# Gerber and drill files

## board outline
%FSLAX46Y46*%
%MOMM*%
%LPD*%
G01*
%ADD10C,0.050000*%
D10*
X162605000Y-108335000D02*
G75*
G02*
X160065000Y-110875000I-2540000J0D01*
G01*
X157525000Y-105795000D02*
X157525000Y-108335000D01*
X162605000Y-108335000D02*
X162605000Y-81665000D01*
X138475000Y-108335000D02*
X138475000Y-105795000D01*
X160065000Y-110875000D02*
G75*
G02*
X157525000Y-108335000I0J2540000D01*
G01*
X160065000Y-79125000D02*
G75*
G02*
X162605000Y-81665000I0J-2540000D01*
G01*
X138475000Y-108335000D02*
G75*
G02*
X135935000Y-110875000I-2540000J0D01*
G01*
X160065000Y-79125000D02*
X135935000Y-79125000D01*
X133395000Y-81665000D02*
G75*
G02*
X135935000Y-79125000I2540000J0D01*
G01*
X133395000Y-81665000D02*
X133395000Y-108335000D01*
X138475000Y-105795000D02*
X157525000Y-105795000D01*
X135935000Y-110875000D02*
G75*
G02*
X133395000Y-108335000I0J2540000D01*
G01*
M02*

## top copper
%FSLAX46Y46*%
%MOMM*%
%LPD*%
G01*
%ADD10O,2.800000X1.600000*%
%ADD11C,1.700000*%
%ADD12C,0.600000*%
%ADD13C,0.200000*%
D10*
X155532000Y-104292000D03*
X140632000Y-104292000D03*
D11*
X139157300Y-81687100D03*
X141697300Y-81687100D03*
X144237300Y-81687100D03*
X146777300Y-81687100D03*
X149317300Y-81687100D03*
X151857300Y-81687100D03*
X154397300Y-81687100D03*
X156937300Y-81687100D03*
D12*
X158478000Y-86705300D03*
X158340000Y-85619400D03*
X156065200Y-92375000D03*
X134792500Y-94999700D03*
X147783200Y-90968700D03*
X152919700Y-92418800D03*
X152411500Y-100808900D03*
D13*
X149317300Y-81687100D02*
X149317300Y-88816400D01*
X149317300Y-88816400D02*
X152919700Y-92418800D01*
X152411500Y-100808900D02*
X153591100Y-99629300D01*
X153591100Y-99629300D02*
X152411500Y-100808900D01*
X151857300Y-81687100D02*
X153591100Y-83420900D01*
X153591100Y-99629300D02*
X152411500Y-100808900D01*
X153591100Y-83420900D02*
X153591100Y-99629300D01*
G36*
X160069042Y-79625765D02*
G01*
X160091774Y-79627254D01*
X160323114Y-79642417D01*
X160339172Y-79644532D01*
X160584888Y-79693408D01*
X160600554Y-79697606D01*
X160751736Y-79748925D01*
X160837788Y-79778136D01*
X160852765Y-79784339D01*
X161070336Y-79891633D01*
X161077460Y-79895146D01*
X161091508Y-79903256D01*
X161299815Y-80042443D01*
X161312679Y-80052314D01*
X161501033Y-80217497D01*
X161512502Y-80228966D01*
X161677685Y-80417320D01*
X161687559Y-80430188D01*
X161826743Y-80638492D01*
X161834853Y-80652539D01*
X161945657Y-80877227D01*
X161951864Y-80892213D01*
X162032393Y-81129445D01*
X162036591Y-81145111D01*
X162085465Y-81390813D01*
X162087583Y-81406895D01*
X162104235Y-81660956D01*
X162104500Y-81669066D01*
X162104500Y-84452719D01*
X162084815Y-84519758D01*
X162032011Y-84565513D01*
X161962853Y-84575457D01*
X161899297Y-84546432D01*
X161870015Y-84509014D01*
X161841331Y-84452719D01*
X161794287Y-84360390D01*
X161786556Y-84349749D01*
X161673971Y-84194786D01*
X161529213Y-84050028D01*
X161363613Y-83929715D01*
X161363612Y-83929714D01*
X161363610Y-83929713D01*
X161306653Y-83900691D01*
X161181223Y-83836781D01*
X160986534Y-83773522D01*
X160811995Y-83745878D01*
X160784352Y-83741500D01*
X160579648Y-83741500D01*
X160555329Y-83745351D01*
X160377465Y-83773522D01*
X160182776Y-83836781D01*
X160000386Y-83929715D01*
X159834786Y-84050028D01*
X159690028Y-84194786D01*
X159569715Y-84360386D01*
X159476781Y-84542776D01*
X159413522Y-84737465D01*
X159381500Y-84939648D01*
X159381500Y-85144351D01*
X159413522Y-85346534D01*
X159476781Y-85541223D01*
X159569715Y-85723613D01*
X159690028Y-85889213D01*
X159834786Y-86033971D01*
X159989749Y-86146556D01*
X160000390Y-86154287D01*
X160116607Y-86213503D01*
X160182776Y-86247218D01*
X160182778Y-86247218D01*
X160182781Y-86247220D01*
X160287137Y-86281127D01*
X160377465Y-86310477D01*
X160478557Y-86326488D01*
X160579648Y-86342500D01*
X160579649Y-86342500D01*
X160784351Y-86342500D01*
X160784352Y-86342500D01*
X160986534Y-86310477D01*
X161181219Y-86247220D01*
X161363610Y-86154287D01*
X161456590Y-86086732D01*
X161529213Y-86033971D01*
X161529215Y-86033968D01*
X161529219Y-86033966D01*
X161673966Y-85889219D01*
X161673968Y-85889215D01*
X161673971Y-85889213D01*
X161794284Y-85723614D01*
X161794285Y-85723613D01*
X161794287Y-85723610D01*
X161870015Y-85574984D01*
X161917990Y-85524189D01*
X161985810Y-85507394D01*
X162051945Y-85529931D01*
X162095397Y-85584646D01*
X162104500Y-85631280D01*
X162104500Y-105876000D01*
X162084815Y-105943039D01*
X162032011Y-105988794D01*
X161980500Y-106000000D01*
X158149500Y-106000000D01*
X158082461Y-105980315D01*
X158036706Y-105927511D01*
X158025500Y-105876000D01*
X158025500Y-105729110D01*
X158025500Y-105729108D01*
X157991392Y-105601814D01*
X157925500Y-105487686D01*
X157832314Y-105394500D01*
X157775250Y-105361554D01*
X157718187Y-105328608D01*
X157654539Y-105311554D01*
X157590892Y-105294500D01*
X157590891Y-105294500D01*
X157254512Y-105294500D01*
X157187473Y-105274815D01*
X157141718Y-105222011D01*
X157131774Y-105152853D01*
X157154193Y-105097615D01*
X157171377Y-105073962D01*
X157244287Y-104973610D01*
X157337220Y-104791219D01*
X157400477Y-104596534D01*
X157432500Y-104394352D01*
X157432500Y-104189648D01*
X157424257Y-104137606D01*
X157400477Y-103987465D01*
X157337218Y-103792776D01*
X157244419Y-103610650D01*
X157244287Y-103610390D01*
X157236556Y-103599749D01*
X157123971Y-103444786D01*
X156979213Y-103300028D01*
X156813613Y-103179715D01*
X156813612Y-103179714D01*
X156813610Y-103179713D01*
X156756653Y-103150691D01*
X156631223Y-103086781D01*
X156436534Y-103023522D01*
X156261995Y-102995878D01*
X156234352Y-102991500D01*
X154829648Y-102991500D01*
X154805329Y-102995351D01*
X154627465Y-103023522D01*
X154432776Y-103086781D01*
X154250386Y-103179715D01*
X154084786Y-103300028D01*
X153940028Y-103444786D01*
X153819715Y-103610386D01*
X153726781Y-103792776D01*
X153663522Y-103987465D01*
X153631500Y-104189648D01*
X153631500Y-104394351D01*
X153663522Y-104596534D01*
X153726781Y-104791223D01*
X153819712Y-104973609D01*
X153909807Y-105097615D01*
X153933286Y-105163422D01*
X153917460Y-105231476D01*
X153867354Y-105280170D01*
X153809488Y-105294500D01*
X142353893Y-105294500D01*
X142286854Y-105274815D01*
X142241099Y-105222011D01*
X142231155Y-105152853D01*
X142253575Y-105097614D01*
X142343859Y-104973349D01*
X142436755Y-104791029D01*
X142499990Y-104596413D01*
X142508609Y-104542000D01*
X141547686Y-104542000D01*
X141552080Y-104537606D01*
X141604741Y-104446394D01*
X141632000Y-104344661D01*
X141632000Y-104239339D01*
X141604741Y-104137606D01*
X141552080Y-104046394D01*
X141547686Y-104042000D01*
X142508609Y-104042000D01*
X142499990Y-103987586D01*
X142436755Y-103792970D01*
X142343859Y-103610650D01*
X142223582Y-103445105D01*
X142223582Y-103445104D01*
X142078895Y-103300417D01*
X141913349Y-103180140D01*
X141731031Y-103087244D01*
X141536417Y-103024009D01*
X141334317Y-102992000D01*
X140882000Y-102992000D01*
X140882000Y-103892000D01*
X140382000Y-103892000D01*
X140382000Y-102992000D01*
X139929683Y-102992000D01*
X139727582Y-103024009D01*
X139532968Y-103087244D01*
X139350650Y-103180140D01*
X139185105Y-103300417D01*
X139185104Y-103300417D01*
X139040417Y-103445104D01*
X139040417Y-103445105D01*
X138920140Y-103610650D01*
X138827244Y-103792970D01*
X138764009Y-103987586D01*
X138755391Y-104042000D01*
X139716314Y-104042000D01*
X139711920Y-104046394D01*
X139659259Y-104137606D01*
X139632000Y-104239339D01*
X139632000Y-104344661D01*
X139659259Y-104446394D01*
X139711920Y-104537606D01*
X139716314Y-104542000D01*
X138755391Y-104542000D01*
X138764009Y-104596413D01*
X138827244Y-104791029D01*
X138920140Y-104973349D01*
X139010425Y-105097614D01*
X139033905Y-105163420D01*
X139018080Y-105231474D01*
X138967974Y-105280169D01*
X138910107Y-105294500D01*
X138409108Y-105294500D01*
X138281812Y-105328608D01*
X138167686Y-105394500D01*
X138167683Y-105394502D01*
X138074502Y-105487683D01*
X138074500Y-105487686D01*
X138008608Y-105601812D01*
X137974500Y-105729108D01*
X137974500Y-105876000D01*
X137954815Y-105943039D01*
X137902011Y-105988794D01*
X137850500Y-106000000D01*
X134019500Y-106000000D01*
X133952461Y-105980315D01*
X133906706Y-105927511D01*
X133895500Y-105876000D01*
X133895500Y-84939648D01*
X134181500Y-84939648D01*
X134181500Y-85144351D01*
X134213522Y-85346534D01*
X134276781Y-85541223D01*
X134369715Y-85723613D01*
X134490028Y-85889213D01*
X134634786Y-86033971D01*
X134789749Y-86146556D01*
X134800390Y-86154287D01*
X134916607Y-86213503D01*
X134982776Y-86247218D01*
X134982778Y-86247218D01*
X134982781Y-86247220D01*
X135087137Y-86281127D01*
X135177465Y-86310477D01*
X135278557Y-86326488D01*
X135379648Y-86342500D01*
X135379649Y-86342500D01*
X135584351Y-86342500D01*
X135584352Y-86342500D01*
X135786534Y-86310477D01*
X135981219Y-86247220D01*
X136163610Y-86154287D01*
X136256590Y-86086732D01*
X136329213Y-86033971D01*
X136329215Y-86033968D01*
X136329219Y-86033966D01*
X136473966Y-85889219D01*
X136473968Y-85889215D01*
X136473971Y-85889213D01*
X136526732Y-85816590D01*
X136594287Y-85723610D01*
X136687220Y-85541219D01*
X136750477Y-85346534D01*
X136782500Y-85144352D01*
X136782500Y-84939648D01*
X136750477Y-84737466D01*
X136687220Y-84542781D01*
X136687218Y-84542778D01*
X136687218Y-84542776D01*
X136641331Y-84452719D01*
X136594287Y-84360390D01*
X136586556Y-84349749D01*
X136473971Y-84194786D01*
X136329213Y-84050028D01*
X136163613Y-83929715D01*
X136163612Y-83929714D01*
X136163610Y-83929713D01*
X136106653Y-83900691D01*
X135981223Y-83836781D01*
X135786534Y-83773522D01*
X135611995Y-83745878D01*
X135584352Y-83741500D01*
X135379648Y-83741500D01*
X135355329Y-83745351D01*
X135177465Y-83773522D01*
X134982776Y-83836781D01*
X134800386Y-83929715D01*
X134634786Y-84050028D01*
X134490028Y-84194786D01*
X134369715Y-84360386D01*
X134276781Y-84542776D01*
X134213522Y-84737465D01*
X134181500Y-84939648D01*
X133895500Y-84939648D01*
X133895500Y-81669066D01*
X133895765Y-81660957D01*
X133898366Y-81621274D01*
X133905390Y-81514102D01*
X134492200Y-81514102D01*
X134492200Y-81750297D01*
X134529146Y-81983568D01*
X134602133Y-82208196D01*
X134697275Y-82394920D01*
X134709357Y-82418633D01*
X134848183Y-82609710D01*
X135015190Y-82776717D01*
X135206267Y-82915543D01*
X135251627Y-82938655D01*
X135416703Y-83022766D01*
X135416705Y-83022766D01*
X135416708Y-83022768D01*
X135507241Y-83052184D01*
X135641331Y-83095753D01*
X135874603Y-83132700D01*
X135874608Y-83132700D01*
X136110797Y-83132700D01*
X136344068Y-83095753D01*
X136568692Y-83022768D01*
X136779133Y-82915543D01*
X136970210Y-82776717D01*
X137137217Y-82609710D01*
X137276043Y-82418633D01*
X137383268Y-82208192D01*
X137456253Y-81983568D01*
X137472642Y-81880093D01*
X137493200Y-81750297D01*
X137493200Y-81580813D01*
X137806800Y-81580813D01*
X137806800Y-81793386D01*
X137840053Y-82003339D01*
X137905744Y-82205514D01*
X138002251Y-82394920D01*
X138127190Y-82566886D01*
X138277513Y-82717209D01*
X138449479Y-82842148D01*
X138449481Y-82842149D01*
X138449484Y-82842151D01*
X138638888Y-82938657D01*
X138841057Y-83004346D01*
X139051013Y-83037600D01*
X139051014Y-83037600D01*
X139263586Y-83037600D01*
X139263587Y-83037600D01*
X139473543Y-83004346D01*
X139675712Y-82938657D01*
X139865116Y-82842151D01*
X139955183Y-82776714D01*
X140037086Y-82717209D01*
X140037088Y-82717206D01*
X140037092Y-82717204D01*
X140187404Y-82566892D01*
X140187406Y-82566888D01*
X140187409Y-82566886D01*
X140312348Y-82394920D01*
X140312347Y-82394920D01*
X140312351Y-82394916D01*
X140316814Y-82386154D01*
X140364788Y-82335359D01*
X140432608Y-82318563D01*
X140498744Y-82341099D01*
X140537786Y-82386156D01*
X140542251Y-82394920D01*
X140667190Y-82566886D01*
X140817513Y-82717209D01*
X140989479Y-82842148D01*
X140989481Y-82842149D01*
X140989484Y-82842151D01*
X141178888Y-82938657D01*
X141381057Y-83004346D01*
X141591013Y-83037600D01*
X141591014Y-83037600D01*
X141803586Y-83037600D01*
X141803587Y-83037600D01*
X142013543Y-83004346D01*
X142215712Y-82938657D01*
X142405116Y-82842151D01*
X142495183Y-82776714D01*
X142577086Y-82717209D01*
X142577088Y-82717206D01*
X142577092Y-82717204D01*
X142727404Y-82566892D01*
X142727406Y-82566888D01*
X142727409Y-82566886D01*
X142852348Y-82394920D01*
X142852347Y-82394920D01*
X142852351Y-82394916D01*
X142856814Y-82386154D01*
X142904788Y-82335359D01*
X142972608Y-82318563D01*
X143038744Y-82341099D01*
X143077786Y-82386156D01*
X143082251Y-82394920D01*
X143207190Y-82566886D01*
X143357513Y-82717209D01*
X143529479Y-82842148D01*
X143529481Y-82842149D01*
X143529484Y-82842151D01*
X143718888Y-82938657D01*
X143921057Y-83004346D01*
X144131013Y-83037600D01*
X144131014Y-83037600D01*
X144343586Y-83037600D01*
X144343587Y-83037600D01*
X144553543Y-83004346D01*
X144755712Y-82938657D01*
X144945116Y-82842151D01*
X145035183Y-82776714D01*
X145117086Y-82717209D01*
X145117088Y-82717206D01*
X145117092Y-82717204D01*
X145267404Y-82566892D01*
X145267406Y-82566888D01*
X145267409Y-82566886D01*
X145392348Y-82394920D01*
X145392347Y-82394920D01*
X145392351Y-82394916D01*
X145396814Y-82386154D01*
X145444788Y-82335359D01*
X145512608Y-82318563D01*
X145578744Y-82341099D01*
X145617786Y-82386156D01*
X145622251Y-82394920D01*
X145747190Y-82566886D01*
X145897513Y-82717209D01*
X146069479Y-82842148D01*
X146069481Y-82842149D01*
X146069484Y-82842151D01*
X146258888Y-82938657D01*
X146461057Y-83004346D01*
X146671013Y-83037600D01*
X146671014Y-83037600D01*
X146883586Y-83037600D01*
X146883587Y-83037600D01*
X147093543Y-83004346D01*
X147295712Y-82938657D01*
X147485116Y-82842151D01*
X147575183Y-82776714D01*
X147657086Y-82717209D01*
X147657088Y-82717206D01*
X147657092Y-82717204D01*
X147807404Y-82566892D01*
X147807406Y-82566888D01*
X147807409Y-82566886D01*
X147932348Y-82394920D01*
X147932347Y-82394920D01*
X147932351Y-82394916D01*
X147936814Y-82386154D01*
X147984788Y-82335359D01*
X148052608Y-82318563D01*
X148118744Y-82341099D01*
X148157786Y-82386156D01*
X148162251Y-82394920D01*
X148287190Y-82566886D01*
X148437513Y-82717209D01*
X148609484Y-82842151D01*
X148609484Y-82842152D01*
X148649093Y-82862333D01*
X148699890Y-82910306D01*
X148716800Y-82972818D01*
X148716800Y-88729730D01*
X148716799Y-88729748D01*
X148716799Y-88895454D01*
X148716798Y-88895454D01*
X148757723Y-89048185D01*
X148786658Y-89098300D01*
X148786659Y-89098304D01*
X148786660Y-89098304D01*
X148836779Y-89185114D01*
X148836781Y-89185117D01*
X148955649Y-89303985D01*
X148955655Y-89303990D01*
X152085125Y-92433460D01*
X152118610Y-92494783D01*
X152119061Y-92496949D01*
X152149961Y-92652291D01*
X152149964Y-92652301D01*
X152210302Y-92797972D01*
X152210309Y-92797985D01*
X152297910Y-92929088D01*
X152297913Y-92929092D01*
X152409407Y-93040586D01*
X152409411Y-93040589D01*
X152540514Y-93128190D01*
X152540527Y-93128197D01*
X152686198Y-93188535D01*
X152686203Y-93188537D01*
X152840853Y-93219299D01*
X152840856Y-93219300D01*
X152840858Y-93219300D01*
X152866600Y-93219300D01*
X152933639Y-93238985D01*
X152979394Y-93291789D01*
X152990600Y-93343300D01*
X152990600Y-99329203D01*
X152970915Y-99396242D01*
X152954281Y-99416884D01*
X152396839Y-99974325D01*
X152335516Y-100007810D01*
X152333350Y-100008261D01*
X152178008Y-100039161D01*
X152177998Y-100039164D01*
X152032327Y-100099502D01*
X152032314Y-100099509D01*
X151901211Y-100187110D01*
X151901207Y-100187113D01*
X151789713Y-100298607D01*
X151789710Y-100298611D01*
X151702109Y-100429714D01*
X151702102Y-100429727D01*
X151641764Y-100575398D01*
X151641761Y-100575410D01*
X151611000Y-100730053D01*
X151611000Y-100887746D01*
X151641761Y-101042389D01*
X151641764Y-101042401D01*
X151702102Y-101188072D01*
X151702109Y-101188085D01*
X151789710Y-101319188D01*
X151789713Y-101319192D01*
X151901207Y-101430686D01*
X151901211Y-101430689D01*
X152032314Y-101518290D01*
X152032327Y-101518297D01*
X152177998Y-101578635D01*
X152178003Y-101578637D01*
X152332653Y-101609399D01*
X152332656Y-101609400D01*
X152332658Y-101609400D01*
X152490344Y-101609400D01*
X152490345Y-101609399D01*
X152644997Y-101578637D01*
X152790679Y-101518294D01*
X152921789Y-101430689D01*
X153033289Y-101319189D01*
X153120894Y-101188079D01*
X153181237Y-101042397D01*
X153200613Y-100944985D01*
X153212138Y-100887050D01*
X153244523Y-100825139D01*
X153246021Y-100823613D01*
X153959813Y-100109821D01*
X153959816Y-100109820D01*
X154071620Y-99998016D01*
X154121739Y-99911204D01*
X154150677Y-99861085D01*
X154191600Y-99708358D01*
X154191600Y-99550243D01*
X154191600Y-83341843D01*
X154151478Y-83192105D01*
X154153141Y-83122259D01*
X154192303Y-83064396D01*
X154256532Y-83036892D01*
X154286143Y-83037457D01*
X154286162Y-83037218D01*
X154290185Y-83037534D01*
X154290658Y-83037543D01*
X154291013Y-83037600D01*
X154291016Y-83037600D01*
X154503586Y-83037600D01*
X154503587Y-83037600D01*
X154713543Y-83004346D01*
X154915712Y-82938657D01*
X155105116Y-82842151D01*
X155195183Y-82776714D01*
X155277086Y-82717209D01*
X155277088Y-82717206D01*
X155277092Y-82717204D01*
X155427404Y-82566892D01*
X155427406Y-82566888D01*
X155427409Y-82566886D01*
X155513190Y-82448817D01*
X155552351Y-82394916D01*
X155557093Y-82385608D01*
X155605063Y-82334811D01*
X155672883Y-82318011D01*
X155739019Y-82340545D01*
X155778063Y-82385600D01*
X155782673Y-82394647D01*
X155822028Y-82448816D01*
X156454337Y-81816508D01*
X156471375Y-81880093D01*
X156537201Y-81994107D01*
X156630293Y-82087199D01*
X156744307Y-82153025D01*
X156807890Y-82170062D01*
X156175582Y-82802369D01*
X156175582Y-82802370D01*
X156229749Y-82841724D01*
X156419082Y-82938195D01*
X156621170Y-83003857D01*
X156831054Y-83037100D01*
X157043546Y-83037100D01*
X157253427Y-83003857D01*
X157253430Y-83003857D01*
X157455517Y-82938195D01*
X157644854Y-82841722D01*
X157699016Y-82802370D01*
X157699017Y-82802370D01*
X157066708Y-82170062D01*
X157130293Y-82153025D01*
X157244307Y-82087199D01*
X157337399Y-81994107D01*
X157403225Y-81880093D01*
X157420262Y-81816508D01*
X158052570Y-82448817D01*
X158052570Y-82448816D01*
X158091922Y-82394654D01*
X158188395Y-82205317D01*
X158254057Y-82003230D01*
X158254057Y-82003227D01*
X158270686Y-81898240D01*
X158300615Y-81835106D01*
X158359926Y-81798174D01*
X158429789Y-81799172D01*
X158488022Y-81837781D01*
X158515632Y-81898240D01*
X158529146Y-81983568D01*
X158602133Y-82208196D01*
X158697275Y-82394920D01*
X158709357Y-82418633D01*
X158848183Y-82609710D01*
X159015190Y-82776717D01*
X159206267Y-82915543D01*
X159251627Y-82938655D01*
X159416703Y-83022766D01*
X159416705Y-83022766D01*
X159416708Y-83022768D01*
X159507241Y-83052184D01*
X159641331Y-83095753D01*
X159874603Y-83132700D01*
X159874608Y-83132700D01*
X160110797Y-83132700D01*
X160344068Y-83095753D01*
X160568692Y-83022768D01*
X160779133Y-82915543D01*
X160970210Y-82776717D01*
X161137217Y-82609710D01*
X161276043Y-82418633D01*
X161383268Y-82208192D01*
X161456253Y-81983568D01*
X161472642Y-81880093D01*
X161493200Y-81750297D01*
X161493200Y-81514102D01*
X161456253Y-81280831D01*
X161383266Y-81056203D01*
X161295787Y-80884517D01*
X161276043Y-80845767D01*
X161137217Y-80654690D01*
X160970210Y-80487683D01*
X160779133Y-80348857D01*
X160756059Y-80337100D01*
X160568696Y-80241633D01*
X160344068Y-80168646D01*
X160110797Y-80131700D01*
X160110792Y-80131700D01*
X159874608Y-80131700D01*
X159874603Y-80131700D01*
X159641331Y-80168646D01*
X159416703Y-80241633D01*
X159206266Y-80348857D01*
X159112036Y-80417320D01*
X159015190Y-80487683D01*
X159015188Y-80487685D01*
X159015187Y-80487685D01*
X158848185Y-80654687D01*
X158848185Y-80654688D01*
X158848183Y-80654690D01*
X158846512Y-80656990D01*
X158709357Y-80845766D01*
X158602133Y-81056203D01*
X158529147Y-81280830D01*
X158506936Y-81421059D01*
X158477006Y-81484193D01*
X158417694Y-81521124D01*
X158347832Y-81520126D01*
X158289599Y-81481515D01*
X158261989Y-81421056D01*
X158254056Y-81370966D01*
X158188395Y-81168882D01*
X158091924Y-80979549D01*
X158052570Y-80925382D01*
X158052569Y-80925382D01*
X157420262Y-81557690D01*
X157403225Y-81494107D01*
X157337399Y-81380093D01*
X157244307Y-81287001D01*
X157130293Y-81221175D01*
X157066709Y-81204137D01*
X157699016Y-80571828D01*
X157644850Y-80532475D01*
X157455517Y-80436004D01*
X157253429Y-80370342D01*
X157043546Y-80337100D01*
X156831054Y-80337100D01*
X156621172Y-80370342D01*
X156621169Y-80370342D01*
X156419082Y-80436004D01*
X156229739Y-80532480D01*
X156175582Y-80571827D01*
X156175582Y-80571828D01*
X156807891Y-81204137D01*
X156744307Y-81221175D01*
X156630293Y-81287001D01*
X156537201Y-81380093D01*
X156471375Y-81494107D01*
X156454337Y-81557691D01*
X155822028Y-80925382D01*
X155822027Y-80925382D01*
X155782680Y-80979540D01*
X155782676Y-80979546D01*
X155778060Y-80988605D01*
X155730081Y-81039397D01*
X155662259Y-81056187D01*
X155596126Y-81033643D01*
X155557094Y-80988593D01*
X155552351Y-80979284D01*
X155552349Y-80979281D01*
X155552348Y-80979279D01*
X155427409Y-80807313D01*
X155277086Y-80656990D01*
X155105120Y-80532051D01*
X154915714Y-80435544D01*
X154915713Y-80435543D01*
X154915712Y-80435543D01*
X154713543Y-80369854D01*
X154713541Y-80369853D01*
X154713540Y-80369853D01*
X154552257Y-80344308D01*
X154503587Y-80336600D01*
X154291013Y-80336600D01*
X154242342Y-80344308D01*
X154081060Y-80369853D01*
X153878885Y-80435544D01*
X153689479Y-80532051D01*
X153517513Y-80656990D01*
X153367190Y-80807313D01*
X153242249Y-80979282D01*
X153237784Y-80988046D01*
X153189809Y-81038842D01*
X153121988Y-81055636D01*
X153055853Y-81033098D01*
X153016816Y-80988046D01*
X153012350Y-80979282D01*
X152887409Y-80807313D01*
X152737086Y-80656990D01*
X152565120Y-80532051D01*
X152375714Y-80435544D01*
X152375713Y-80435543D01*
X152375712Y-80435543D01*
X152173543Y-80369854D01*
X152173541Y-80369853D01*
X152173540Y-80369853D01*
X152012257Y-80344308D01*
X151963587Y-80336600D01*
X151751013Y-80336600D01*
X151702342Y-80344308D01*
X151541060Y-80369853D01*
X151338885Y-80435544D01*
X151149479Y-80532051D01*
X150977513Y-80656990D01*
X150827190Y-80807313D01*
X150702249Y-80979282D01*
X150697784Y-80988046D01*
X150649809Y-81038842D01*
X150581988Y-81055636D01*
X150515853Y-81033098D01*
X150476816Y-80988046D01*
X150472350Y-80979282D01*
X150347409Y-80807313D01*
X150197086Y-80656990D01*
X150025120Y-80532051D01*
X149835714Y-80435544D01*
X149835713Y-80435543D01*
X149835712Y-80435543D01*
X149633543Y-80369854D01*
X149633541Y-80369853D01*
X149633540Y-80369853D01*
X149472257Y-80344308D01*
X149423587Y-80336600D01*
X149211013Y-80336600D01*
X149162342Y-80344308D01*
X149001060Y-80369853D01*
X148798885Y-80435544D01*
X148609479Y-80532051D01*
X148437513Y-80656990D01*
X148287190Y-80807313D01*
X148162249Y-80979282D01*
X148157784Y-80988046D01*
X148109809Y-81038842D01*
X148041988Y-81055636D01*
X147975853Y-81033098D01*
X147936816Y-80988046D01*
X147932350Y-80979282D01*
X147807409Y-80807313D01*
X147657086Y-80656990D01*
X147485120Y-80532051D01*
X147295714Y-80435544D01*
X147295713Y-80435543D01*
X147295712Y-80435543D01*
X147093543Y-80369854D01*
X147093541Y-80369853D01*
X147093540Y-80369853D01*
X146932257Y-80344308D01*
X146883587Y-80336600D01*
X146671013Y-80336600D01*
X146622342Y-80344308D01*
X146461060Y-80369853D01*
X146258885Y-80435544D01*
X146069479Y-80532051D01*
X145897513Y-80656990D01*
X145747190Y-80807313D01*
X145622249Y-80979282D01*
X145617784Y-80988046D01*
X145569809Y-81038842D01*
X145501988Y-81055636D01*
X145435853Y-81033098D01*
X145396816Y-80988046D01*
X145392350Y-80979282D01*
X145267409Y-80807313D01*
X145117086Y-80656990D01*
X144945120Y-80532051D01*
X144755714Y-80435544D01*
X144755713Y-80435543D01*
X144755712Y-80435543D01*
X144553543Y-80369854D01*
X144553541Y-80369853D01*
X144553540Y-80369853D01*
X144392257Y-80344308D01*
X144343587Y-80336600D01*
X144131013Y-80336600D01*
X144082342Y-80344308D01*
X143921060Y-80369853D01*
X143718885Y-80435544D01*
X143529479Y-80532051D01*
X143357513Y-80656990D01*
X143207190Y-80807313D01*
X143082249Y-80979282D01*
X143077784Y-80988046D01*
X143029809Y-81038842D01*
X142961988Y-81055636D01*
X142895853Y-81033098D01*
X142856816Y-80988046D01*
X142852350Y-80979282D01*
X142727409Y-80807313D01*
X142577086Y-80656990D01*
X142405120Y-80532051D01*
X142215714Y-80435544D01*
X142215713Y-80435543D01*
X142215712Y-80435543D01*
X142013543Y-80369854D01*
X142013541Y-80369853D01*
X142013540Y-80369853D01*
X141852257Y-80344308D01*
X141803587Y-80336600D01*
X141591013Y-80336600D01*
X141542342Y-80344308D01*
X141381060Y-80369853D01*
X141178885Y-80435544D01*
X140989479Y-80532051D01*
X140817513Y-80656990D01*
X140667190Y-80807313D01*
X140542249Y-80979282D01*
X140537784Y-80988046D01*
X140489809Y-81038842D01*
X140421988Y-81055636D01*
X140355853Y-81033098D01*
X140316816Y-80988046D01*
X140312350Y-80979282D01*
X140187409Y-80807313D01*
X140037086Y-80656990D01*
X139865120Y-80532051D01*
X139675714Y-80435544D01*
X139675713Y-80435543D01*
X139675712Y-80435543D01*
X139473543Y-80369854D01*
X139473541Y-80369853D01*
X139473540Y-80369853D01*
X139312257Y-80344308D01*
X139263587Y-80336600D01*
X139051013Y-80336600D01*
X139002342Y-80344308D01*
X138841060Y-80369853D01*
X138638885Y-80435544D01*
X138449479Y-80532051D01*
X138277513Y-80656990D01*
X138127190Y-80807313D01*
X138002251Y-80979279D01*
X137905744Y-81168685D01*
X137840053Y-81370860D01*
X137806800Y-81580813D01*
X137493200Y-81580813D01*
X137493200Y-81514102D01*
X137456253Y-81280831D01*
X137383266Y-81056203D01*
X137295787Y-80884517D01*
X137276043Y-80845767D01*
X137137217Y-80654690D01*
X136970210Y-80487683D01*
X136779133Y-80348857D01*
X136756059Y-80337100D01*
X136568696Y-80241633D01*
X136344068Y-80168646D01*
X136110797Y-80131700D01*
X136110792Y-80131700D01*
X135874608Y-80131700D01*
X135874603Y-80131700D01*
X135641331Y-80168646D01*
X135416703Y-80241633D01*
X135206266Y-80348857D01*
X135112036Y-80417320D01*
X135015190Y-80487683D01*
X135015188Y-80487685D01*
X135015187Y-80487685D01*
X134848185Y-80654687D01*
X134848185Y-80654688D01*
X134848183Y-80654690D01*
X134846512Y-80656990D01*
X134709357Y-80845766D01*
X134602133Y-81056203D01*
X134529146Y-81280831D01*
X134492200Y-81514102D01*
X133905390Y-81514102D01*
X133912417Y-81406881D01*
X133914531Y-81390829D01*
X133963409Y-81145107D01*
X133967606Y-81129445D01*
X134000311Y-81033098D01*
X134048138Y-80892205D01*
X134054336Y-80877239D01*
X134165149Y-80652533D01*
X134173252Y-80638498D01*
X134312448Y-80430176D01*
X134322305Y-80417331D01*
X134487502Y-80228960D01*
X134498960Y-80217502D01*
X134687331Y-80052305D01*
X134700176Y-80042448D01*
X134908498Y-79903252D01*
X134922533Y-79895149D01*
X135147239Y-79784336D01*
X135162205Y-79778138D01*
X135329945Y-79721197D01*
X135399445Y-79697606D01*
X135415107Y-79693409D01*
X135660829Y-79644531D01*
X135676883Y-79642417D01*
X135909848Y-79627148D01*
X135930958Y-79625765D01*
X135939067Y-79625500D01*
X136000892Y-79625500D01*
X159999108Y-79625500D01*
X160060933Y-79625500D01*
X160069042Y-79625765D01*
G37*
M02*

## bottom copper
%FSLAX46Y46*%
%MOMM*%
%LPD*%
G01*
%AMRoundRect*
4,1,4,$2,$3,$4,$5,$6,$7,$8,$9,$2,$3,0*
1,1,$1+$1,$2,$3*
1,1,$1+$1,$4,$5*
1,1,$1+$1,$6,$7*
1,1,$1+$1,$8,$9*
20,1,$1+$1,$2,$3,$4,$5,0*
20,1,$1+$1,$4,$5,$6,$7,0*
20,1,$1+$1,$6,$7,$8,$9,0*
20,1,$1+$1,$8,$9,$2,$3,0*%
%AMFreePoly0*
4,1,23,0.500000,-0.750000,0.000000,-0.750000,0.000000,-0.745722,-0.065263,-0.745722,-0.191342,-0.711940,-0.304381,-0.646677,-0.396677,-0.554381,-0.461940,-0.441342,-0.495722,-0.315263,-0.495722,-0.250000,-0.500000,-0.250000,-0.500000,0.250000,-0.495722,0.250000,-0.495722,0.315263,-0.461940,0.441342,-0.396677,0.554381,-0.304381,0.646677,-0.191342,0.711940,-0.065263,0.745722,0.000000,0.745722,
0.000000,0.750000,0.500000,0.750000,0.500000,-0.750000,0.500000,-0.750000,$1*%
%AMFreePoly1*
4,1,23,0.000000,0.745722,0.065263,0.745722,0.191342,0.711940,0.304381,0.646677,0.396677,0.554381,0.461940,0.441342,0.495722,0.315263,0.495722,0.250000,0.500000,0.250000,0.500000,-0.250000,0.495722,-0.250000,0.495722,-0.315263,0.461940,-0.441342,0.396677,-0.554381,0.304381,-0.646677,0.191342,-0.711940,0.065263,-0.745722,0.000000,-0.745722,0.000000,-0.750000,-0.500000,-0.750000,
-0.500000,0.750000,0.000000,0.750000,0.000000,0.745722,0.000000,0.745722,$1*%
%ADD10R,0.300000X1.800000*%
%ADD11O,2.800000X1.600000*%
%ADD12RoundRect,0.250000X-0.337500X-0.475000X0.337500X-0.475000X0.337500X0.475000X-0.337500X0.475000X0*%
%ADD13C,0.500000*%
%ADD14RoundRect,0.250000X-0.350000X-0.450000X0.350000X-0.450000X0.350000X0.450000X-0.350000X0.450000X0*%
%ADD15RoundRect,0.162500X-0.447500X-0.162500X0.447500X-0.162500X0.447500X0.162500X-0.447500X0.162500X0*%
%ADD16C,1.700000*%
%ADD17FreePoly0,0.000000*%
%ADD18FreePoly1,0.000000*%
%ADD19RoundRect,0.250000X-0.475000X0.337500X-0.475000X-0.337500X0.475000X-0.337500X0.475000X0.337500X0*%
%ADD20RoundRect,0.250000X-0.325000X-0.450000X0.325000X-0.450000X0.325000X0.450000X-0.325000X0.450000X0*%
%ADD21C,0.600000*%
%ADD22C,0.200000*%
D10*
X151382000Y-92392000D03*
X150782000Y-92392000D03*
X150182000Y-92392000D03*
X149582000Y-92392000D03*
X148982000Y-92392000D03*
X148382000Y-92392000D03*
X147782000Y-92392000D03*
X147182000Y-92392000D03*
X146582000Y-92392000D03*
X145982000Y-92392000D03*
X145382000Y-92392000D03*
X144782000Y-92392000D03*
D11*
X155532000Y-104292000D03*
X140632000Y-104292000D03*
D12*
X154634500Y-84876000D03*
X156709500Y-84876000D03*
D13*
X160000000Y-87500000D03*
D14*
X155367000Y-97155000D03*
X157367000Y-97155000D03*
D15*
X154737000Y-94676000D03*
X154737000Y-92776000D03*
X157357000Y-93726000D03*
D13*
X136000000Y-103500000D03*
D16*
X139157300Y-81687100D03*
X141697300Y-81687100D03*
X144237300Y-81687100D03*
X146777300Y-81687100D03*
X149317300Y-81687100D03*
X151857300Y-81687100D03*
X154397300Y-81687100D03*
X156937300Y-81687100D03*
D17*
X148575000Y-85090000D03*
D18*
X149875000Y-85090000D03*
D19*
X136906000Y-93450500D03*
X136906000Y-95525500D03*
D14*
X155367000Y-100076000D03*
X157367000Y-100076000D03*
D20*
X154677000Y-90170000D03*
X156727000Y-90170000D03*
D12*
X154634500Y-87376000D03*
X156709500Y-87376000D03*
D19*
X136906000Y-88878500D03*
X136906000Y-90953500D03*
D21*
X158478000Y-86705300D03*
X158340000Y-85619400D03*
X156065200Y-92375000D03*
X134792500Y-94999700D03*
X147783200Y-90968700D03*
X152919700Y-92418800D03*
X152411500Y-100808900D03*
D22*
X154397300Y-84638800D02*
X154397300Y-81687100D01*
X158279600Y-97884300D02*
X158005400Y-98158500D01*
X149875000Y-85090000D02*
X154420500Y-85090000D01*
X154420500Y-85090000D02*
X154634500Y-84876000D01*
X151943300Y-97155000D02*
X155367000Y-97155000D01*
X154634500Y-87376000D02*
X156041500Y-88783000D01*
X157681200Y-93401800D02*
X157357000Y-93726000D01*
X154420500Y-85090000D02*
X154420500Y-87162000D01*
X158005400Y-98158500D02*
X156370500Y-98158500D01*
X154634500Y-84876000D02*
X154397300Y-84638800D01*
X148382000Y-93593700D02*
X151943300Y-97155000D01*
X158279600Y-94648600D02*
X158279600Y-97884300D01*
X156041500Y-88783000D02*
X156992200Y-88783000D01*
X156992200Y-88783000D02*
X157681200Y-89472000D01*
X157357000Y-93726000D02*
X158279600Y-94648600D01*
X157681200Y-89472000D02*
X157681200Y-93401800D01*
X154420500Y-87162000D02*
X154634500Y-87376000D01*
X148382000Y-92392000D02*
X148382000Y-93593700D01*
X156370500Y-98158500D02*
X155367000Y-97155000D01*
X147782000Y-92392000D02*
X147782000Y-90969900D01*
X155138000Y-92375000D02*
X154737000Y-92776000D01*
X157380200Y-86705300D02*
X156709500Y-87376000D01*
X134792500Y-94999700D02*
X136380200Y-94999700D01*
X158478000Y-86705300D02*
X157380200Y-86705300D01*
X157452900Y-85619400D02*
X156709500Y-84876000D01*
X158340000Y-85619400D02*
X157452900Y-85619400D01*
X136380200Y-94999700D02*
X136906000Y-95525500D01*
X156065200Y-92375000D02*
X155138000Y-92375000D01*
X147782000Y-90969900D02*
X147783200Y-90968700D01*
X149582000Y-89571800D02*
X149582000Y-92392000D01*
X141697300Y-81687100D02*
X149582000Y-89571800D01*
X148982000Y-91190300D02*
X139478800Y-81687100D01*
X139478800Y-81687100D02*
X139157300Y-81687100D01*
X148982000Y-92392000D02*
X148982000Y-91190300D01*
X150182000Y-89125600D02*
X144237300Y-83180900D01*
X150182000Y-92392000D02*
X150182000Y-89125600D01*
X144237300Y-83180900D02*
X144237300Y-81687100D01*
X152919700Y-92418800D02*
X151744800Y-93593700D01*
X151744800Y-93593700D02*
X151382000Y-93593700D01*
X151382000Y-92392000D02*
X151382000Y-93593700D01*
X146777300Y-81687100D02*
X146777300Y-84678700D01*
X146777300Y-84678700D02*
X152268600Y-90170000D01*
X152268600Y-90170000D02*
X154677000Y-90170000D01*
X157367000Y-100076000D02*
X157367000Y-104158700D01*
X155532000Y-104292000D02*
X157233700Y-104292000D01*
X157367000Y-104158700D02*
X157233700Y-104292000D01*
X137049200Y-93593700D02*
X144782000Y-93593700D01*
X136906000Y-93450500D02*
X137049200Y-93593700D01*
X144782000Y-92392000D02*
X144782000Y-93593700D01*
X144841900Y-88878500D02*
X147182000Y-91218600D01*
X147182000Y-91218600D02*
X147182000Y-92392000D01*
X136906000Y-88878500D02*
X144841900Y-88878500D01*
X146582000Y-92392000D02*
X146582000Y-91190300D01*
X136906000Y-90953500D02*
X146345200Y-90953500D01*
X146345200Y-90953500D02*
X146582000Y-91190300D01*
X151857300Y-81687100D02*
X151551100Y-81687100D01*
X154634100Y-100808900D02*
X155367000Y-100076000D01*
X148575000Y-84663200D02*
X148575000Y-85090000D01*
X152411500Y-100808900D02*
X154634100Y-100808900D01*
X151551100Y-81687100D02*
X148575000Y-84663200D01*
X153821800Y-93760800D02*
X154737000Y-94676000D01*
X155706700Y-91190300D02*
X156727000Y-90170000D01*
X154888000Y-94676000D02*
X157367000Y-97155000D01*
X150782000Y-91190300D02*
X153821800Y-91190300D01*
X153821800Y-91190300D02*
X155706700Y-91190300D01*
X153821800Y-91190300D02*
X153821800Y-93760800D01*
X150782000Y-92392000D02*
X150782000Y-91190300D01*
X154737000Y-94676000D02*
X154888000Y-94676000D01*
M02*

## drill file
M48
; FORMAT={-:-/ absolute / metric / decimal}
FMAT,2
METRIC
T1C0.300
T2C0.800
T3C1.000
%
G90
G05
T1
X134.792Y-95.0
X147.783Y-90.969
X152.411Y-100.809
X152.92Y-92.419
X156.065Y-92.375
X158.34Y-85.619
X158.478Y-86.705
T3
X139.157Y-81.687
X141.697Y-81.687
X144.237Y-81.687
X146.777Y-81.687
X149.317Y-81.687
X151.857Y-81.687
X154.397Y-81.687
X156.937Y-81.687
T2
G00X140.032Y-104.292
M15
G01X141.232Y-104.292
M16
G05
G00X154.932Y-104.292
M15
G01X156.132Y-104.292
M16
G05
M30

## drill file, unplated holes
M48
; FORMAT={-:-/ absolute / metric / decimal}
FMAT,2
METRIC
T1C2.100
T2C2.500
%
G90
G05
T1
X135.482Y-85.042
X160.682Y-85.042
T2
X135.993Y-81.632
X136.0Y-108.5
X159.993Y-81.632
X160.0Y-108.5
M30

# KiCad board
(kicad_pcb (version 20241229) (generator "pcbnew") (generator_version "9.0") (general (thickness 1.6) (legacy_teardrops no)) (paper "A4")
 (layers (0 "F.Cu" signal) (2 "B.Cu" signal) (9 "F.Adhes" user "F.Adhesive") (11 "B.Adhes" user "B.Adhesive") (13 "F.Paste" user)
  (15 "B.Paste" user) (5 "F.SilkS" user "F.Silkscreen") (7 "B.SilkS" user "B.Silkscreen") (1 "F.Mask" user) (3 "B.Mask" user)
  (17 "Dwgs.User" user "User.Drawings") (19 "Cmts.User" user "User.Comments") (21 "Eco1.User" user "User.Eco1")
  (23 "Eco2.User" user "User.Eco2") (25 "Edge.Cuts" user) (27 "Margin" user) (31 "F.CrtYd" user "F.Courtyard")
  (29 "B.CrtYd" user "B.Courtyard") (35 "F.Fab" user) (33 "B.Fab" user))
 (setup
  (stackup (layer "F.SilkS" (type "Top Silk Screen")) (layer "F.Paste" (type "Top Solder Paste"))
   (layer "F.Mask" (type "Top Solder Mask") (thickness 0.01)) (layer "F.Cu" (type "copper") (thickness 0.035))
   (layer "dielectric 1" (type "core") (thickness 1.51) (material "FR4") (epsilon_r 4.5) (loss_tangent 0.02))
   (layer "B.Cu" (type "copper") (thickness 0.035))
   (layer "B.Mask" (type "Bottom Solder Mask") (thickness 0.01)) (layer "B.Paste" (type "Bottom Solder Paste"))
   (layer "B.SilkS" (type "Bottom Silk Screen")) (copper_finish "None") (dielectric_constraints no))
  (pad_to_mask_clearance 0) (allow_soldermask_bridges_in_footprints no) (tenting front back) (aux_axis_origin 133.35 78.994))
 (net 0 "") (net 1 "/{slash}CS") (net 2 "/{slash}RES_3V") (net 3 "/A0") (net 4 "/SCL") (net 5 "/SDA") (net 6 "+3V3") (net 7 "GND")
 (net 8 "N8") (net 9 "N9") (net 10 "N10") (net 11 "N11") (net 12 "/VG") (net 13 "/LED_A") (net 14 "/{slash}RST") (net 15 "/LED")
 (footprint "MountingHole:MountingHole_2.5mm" (layer "F.Cu") (at 160 108.5)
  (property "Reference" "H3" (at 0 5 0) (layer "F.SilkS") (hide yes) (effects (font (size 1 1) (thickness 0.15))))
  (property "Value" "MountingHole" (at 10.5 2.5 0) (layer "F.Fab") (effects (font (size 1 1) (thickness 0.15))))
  (pad "" np_thru_hole circle (at 0 0) (size 2.5 2.5) (drill 2.5) (layers "*.Cu" "*.Mask")))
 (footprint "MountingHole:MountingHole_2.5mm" (layer "F.Cu") (at 159.9927 81.6322)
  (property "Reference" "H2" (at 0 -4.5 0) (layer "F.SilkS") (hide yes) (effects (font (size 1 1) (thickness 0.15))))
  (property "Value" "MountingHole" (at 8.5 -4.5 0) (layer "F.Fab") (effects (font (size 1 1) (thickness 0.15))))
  (pad "" np_thru_hole circle (at 0 0) (size 2.5 2.5) (drill 2.5) (layers "*.Cu" "*.Mask")))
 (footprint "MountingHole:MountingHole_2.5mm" (layer "F.Cu") (at 135.9927 81.6322)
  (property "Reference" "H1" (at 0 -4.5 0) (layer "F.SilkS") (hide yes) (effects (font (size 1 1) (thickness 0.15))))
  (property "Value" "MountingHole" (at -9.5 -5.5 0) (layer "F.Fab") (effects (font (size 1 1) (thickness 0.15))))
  (pad "" np_thru_hole circle (at 0 0) (size 2.5 2.5) (drill 2.5) (layers "*.Cu" "*.Mask")))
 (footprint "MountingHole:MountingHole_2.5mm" (layer "F.Cu") (at 136 108.5)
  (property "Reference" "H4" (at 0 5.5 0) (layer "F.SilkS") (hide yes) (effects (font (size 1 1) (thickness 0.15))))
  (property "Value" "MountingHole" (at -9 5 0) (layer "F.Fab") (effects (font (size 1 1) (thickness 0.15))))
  (pad "" np_thru_hole circle (at 0 0) (size 2.5 2.5) (drill 2.5) (layers "*.Cu" "*.Mask")))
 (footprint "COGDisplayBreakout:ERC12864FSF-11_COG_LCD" (layer "F.Cu") (at 148.082 94.742)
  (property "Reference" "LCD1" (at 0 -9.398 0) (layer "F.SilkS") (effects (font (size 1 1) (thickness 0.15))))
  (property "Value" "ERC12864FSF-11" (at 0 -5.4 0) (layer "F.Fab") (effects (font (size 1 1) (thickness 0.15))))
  (pad "" np_thru_hole circle (at -12.6 -9.7) (size 2.1 2.1) (drill 2.1) (layers "*.Cu" "*.Mask"))
  (pad "" np_thru_hole circle (at 12.6 -9.7) (size 2.1 2.1) (drill 2.1) (layers "*.Cu" "*.Mask"))
  (pad "1" smd rect (at 3.3 -2.35) (size 0.3 1.8) (layers "B.Cu" "B.Mask" "B.Paste") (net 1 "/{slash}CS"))
  (pad "2" smd rect (at 2.7 -2.35) (size 0.3 1.8) (layers "B.Cu" "B.Mask" "B.Paste") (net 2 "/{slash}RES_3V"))
  (pad "3" smd rect (at 2.1 -2.35) (size 0.3 1.8) (layers "B.Cu" "B.Mask" "B.Paste") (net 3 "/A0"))
  (pad "4" smd rect (at 1.5 -2.35) (size 0.3 1.8) (layers "B.Cu" "B.Mask" "B.Paste") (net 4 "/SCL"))
  (pad "5" smd rect (at 0.9 -2.35) (size 0.3 1.8) (layers "B.Cu" "B.Mask" "B.Paste") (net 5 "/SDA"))
  (pad "6" smd rect (at 0.3 -2.35) (size 0.3 1.8) (layers "B.Cu" "B.Mask" "B.Paste") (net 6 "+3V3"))
  (pad "7" smd rect (at -0.3 -2.35) (size 0.3 1.8) (layers "B.Cu" "B.Mask" "B.Paste") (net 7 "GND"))
  (pad "8" smd rect (at -0.9 -2.35) (size 0.3 1.8) (layers "B.Cu" "B.Mask" "B.Paste") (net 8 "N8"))
  (pad "9" smd rect (at -1.5 -2.35) (size 0.3 1.8) (layers "B.Cu" "B.Mask" "B.Paste") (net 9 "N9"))
  (pad "10" smd rect (at -2.1 -2.35) (size 0.3 1.8) (layers "B.Cu" "B.Mask" "B.Paste") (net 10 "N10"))
  (pad "11" smd rect (at -2.7 -2.35) (size 0.3 1.8) (layers "B.Cu" "B.Mask" "B.Paste") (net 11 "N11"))
  (pad "12" smd rect (at -3.3 -2.35) (size 0.3 1.8) (layers "B.Cu" "B.Mask" "B.Paste") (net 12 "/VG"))
  (pad "A" thru_hole oval (at 7.45 9.55) (size 2.8 1.6) (drill oval 2 0.8) (layers "*.Cu" "*.Mask") (remove_unused_layers no)
   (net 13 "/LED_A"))
  (pad "K" thru_hole oval (at -7.45 9.55) (size 2.8 1.6) (drill oval 2 0.8) (layers "*.Cu" "*.Mask") (remove_unused_layers no) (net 7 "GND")))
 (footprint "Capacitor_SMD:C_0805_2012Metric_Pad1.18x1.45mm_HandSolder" (layer "B.Cu") (at 155.672 84.876)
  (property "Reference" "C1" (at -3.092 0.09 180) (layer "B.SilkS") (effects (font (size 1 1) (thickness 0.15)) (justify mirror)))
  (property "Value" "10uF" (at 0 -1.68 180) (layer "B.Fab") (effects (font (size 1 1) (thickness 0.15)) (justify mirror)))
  (pad "1" smd roundrect (at -1.0375 0) (size 1.175 1.45) (layers "B.Cu" "B.Mask" "B.Paste") (roundrect_rratio 0.212766) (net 6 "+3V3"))
  (pad "2" smd roundrect (at 1.0375 0) (size 1.175 1.45) (layers "B.Cu" "B.Mask" "B.Paste") (roundrect_rratio 0.212766) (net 7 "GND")))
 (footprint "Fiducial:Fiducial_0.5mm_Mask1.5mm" (layer "B.Cu") (at 160 87.5 180)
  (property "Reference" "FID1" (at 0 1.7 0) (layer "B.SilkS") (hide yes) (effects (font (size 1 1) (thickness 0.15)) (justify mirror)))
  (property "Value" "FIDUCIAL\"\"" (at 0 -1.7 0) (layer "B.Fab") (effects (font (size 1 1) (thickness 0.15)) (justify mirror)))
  (pad "" smd circle (at 0 0 180) (size 0.5 0.5) (layers "B.Cu" "B.Mask") (solder_mask_margin 0.5) (clearance 0.6)))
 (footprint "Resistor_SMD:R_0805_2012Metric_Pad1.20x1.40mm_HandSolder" (layer "B.Cu") (at 156.367 97.155)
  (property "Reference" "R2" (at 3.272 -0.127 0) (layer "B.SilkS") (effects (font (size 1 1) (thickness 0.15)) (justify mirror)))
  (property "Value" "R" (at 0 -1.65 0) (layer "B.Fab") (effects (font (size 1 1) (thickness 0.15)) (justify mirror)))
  (pad "1" smd roundrect (at -1 0) (size 1.2 1.4) (layers "B.Cu" "B.Mask" "B.Paste") (roundrect_rratio 0.208333) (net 6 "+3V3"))
  (pad "2" smd roundrect (at 1 0) (size 1.2 1.4) (layers "B.Cu" "B.Mask" "B.Paste") (roundrect_rratio 0.208333) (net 2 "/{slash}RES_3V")))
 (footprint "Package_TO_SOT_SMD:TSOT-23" (layer "B.Cu") (at 156.047 93.726)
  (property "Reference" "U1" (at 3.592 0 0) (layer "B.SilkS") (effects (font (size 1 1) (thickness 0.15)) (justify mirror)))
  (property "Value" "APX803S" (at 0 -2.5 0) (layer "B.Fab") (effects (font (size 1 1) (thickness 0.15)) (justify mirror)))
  (pad "1" smd roundrect (at -1.31 0.95) (size 1.22 0.65) (layers "B.Cu" "B.Mask" "B.Paste") (roundrect_rratio 0.25)
   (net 2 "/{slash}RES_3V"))
  (pad "2" smd roundrect (at -1.31 -0.95) (size 1.22 0.65) (layers "B.Cu" "B.Mask" "B.Paste") (roundrect_rratio 0.25) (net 7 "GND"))
  (pad "3" smd roundrect (at 1.31 0) (size 1.22 0.65) (layers "B.Cu" "B.Mask" "B.Paste") (roundrect_rratio 0.25) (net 6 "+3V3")))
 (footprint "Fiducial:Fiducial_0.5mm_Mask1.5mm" (layer "B.Cu") (at 136 103.5 180)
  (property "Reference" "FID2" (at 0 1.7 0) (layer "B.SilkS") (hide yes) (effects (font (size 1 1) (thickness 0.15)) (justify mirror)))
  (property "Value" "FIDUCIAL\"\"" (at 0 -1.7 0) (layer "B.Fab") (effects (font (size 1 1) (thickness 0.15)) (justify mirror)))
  (pad "" smd circle (at 0 0 180) (size 0.5 0.5) (layers "B.Cu" "B.Mask") (solder_mask_margin 0.5) (clearance 0.6)))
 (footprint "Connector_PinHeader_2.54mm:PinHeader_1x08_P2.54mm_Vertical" (layer "B.Cu") (at 139.1573 81.6871 -90)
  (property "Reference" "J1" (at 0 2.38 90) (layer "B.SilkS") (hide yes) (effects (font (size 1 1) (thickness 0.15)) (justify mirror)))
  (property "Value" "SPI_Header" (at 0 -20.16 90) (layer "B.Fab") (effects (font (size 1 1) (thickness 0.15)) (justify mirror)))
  (pad "1" thru_hole circle (at 0 0 270) (size 1.7 1.7) (drill 1) (layers "*.Cu" "*.Mask") (remove_unused_layers no) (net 5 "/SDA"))
  (pad "2" thru_hole circle (at 0 -2.54 270) (size 1.7 1.7) (drill 1) (layers "*.Cu" "*.Mask") (remove_unused_layers no) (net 4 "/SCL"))
  (pad "3" thru_hole circle (at 0 -5.08 270) (size 1.7 1.7) (drill 1) (layers "*.Cu" "*.Mask") (remove_unused_layers no) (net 3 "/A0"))
  (pad "4" thru_hole circle (at 0 -7.62 270) (size 1.7 1.7) (drill 1) (layers "*.Cu" "*.Mask") (remove_unused_layers no)
   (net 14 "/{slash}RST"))
  (pad "5" thru_hole circle (at 0 -10.16 270) (size 1.7 1.7) (drill 1) (layers "*.Cu" "*.Mask") (remove_unused_layers no)
   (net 1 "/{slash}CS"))
  (pad "6" thru_hole circle (at 0 -12.7 270) (size 1.7 1.7) (drill 1) (layers "*.Cu" "*.Mask") (remove_unused_layers no) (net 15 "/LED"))
  (pad "7" thru_hole circle (at 0 -15.24 270) (size 1.7 1.7) (drill 1) (layers "*.Cu" "*.Mask") (remove_unused_layers no) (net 6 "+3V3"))
  (pad "8" thru_hole circle (at 0 -17.78 270) (size 1.7 1.7) (drill 1) (layers "*.Cu" "*.Mask") (remove_unused_layers no) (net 7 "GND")))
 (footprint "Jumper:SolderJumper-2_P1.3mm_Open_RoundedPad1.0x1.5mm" (layer "B.Cu") (at 149.225 85.09)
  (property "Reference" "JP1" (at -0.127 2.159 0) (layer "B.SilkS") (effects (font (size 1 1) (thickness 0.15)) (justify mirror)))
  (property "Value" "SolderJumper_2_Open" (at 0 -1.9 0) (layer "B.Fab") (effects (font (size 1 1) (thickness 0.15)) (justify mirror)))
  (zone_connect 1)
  (pad "1" smd custom (at -0.65 0) (size 1 0.5) (layers "B.Cu" "B.Mask") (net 15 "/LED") (zone_connect 2) (thermal_bridge_angle 45)
   (options (clearance outline) (anchor rect)) (primitives))
  (pad "2" smd custom (at 0.65 0) (size 1 0.5) (layers "B.Cu" "B.Mask") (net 6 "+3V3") (zone_connect 2) (thermal_bridge_angle 45)
   (options (clearance outline) (anchor rect)) (primitives)))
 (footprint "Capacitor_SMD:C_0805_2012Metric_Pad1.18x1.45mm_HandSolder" (layer "B.Cu") (at 136.906 94.488 -90)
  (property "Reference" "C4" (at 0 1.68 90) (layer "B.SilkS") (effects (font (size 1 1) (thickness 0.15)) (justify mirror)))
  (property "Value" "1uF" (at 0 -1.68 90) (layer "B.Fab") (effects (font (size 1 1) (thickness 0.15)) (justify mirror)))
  (pad "1" smd roundrect (at -1.0375 0 270) (size 1.175 1.45) (layers "B.Cu" "B.Mask" "B.Paste") (roundrect_rratio 0.212766) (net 12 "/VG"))
  (pad "2" smd roundrect (at 1.0375 0 270) (size 1.175 1.45) (layers "B.Cu" "B.Mask" "B.Paste") (roundrect_rratio 0.212766) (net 7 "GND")))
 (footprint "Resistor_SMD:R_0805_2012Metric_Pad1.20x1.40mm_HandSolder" (layer "B.Cu") (at 156.367 100.076)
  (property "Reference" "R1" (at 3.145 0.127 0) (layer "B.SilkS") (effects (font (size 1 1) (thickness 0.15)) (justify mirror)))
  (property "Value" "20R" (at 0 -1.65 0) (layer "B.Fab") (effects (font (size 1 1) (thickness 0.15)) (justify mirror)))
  (pad "1" smd roundrect (at -1 0) (size 1.2 1.4) (layers "B.Cu" "B.Mask" "B.Paste") (roundrect_rratio 0.208333) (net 15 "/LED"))
  (pad "2" smd roundrect (at 1 0) (size 1.2 1.4) (layers "B.Cu" "B.Mask" "B.Paste") (roundrect_rratio 0.208333) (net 13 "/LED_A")))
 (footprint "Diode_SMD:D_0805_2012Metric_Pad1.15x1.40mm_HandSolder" (layer "B.Cu") (at 155.702 90.17)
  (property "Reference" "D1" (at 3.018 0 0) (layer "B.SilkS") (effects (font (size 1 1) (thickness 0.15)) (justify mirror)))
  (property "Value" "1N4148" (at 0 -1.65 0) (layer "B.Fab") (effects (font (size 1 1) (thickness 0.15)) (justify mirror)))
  (pad "1" smd roundrect (at -1.025 0) (size 1.15 1.4) (layers "B.Cu" "B.Mask" "B.Paste") (roundrect_rratio 0.217391) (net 14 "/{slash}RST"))
  (pad "2" smd roundrect (at 1.025 0) (size 1.15 1.4) (layers "B.Cu" "B.Mask" "B.Paste") (roundrect_rratio 0.217391)
   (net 2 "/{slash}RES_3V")))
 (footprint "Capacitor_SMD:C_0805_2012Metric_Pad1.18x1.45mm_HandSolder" (layer "B.Cu") (at 155.672 87.376)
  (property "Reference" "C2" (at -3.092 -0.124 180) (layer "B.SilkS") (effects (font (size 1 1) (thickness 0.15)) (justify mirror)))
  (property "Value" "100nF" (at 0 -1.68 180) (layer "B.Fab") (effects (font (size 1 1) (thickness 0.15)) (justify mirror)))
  (pad "1" smd roundrect (at -1.0375 0) (size 1.175 1.45) (layers "B.Cu" "B.Mask" "B.Paste") (roundrect_rratio 0.212766) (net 6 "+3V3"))
  (pad "2" smd roundrect (at 1.0375 0) (size 1.175 1.45) (layers "B.Cu" "B.Mask" "B.Paste") (roundrect_rratio 0.212766) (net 7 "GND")))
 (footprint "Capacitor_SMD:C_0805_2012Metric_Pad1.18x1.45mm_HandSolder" (layer "B.Cu") (at 136.906 89.916 -90)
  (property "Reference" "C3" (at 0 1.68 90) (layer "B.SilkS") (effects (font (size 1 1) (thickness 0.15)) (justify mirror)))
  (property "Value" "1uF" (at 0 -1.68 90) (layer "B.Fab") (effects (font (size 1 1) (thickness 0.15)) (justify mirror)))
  (pad "1" smd roundrect (at -1.0375 0 270) (size 1.175 1.45) (layers "B.Cu" "B.Mask" "B.Paste") (roundrect_rratio 0.212766) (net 8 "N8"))
  (pad "2" smd roundrect (at 1.0375 0 270) (size 1.175 1.45) (layers "B.Cu" "B.Mask" "B.Paste") (roundrect_rratio 0.212766) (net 9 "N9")))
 (gr_arc (start 162.605 108.335) (mid 161.861051 110.131051) (end 160.065 110.875) (stroke (width 0.05) (type solid)) (layer "Edge.Cuts"))
 (gr_line (start 157.525 105.795) (end 157.525 108.335) (stroke (width 0.05) (type solid)) (layer "Edge.Cuts"))
 (gr_line (start 162.605 108.335) (end 162.605 81.665) (stroke (width 0.05) (type solid)) (layer "Edge.Cuts"))
 (gr_line (start 138.475 108.335) (end 138.475 105.795) (stroke (width 0.05) (type solid)) (layer "Edge.Cuts"))
 (gr_arc (start 160.065 110.875) (mid 158.268949 110.131051) (end 157.525 108.335) (stroke (width 0.05) (type solid)) (layer "Edge.Cuts"))
 (gr_arc (start 160.065 79.125) (mid 161.861051 79.868949) (end 162.605 81.665) (stroke (width 0.05) (type solid)) (layer "Edge.Cuts"))
 (gr_arc (start 138.475 108.335) (mid 137.731051 110.131051) (end 135.935 110.875) (stroke (width 0.05) (type solid)) (layer "Edge.Cuts"))
 (gr_line (start 160.065 79.125) (end 135.935 79.125) (stroke (width 0.05) (type solid)) (layer "Edge.Cuts"))
 (gr_arc (start 133.395 81.665) (mid 134.138949 79.868949) (end 135.935 79.125) (stroke (width 0.05) (type solid)) (layer "Edge.Cuts"))
 (gr_line (start 133.395 81.665) (end 133.395 108.335) (stroke (width 0.05) (type solid)) (layer "Edge.Cuts"))
 (gr_line (start 138.475 105.795) (end 157.525 105.795) (stroke (width 0.05) (type solid)) (layer "Edge.Cuts"))
 (gr_arc (start 135.935 110.875) (mid 134.138949 110.131051) (end 133.395 108.335) (stroke (width 0.05) (type solid)) (layer "Edge.Cuts"))
 (segment (start 154.3973 84.6388) (end 154.3973 81.6871) (width 0.2) (layer "B.Cu") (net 6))
 (segment (start 158.2796 97.8843) (end 158.0054 98.1585) (width 0.2) (layer "B.Cu") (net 6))
 (segment (start 149.875 85.09) (end 154.4205 85.09) (width 0.2) (layer "B.Cu") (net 6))
 (segment (start 154.4205 85.09) (end 154.6345 84.876) (width 0.2) (layer "B.Cu") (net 6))
 (segment (start 151.9433 97.155) (end 155.367 97.155) (width 0.2) (layer "B.Cu") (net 6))
 (segment (start 154.6345 87.376) (end 156.0415 88.783) (width 0.2) (layer "B.Cu") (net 6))
 (segment (start 157.6812 93.4018) (end 157.357 93.726) (width 0.2) (layer "B.Cu") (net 6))
 (segment (start 154.4205 85.09) (end 154.4205 87.162) (width 0.2) (layer "B.Cu") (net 6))
 (segment (start 158.0054 98.1585) (end 156.3705 98.1585) (width 0.2) (layer "B.Cu") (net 6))
 (segment (start 154.6345 84.876) (end 154.3973 84.6388) (width 0.2) (layer "B.Cu") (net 6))
 (segment (start 148.382 93.5937) (end 151.9433 97.155) (width 0.2) (layer "B.Cu") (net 6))
 (segment (start 158.2796 94.6486) (end 158.2796 97.8843) (width 0.2) (layer "B.Cu") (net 6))
 (segment (start 156.0415 88.783) (end 156.9922 88.783) (width 0.2) (layer "B.Cu") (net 6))
 (segment (start 156.9922 88.783) (end 157.6812 89.472) (width 0.2) (layer "B.Cu") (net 6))
 (segment (start 157.357 93.726) (end 158.2796 94.6486) (width 0.2) (layer "B.Cu") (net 6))
 (segment (start 157.6812 89.472) (end 157.6812 93.4018) (width 0.2) (layer "B.Cu") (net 6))
 (segment (start 154.4205 87.162) (end 154.6345 87.376) (width 0.2) (layer "B.Cu") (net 6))
 (segment (start 148.382 92.392) (end 148.382 93.5937) (width 0.2) (layer "B.Cu") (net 6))
 (segment (start 156.3705 98.1585) (end 155.367 97.155) (width 0.2) (layer "B.Cu") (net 6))
 (via (at 158.478 86.7053) (size 0.6) (drill 0.3) (layers "F.Cu" "B.Cu") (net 7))
 (via (at 158.34 85.6194) (size 0.6) (drill 0.3) (layers "F.Cu" "B.Cu") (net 7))
 (via (at 156.0652 92.375) (size 0.6) (drill 0.3) (layers "F.Cu" "B.Cu") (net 7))
 (via (at 134.7925 94.9997) (size 0.6) (drill 0.3) (layers "F.Cu" "B.Cu") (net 7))
 (via (at 147.7832 90.9687) (size 0.6) (drill 0.3) (layers "F.Cu" "B.Cu") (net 7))
 (segment (start 147.782 92.392) (end 147.782 90.9699) (width 0.2) (layer "B.Cu") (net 7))
 (segment (start 155.138 92.375) (end 154.737 92.776) (width 0.2) (layer "B.Cu") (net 7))
 (segment (start 157.3802 86.7053) (end 156.7095 87.376) (width 0.2) (layer "B.Cu") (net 7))
 (segment (start 134.7925 94.9997) (end 136.3802 94.9997) (width 0.2) (layer "B.Cu") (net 7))
 (segment (start 158.478 86.7053) (end 157.3802 86.7053) (width 0.2) (layer "B.Cu") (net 7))
 (segment (start 157.4529 85.6194) (end 156.7095 84.876) (width 0.2) (layer "B.Cu") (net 7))
 (segment (start 158.34 85.6194) (end 157.4529 85.6194) (width 0.2) (layer "B.Cu") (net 7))
 (segment (start 136.3802 94.9997) (end 136.906 95.5255) (width 0.2) (layer "B.Cu") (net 7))
 (segment (start 156.0652 92.375) (end 155.138 92.375) (width 0.2) (layer "B.Cu") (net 7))
 (segment (start 147.782 90.9699) (end 147.7832 90.9687) (width 0.2) (layer "B.Cu") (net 7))
 (segment (start 149.582 89.5718) (end 149.582 92.392) (width 0.2) (layer "B.Cu") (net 4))
 (segment (start 141.6973 81.6871) (end 149.582 89.5718) (width 0.2) (layer "B.Cu") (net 4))
 (segment (start 148.982 91.1903) (end 139.4788 81.6871) (width 0.2) (layer "B.Cu") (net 5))
 (segment (start 139.4788 81.6871) (end 139.1573 81.6871) (width 0.2) (layer "B.Cu") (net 5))
 (segment (start 148.982 92.392) (end 148.982 91.1903) (width 0.2) (layer "B.Cu") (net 5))
 (segment (start 150.182 89.1256) (end 144.2373 83.1809) (width 0.2) (layer "B.Cu") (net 3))
 (segment (start 150.182 92.392) (end 150.182 89.1256) (width 0.2) (layer "B.Cu") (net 3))
 (segment (start 144.2373 83.1809) (end 144.2373 81.6871) (width 0.2) (layer "B.Cu") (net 3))
 (segment (start 149.3173 81.6871) (end 149.3173 88.8164) (width 0.2) (layer "F.Cu") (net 1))
 (segment (start 149.3173 88.8164) (end 152.9197 92.4188) (width 0.2) (layer "F.Cu") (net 1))
 (via (at 152.9197 92.4188) (size 0.6) (drill 0.3) (layers "F.Cu" "B.Cu") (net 1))
 (segment (start 152.9197 92.4188) (end 151.7448 93.5937) (width 0.2) (layer "B.Cu") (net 1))
 (segment (start 151.7448 93.5937) (end 151.382 93.5937) (width 0.2) (layer "B.Cu") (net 1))
 (segment (start 151.382 92.392) (end 151.382 93.5937) (width 0.2) (layer "B.Cu") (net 1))
 (segment (start 146.7773 81.6871) (end 146.7773 84.6787) (width 0.2) (layer "B.Cu") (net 14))
 (segment (start 146.7773 84.6787) (end 152.2686 90.17) (width 0.2) (layer "B.Cu") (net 14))
 (segment (start 152.2686 90.17) (end 154.677 90.17) (width 0.2) (layer "B.Cu") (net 14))
 (segment (start 157.367 100.076) (end 157.367 104.1587) (width 0.2) (layer "B.Cu") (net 13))
 (segment (start 155.532 104.292) (end 157.2337 104.292) (width 0.2) (layer "B.Cu") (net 13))
 (segment (start 157.367 104.1587) (end 157.2337 104.292) (width 0.2) (layer "B.Cu") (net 13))
 (segment (start 137.0492 93.5937) (end 144.782 93.5937) (width 0.2) (layer "B.Cu") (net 12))
 (segment (start 136.906 93.4505) (end 137.0492 93.5937) (width 0.2) (layer "B.Cu") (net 12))
 (segment (start 144.782 92.392) (end 144.782 93.5937) (width 0.2) (layer "B.Cu") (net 12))
 (segment (start 144.8419 88.8785) (end 147.182 91.2186) (width 0.2) (layer "B.Cu") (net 8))
 (segment (start 147.182 91.2186) (end 147.182 92.392) (width 0.2) (layer "B.Cu") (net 8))
 (segment (start 136.906 88.8785) (end 144.8419 88.8785) (width 0.2) (layer "B.Cu") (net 8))
 (segment (start 146.582 92.392) (end 146.582 91.1903) (width 0.2) (layer "B.Cu") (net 9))
 (segment (start 136.906 90.9535) (end 146.3452 90.9535) (width 0.2) (layer "B.Cu") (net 9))
 (segment (start 146.3452 90.9535) (end 146.582 91.1903) (width 0.2) (layer "B.Cu") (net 9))
 (segment (start 152.4115 100.8089) (end 153.5911 99.6293) (width 0.2) (layer "F.Cu") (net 15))
 (segment (start 153.5911 99.6293) (end 152.4115 100.8089) (width 0.2) (layer "F.Cu") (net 15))
 (segment (start 151.8573 81.6871) (end 153.5911 83.4209) (width 0.2) (layer "F.Cu") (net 15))
 (segment (start 153.5911 99.6293) (end 152.4115 100.8089) (width 0.2) (layer "F.Cu") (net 15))
 (segment (start 153.5911 83.4209) (end 153.5911 99.6293) (width 0.2) (layer "F.Cu") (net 15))
 (via (at 152.4115 100.8089) (size 0.6) (drill 0.3) (layers "F.Cu" "B.Cu") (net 15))
 (segment (start 151.8573 81.6871) (end 151.5511 81.6871) (width 0.2) (layer "B.Cu") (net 15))
 (segment (start 154.6341 100.8089) (end 155.367 100.076) (width 0.2) (layer "B.Cu") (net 15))
 (segment (start 148.575 84.6632) (end 148.575 85.09) (width 0.2) (layer "B.Cu") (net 15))
 (segment (start 152.4115 100.8089) (end 154.6341 100.8089) (width 0.2) (layer "B.Cu") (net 15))
 (segment (start 151.5511 81.6871) (end 148.575 84.6632) (width 0.2) (layer "B.Cu") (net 15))
 (segment (start 153.8218 93.7608) (end 154.737 94.676) (width 0.2) (layer "B.Cu") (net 2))
 (segment (start 155.7067 91.1903) (end 156.727 90.17) (width 0.2) (layer "B.Cu") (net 2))
 (segment (start 154.888 94.676) (end 157.367 97.155) (width 0.2) (layer "B.Cu") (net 2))
 (segment (start 150.782 91.1903) (end 153.8218 91.1903) (width 0.2) (layer "B.Cu") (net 2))
 (segment (start 153.8218 91.1903) (end 155.7067 91.1903) (width 0.2) (layer "B.Cu") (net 2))
 (segment (start 153.8218 91.1903) (end 153.8218 93.7608) (width 0.2) (layer "B.Cu") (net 2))
 (segment (start 150.782 92.392) (end 150.782 91.1903) (width 0.2) (layer "B.Cu") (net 2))
 (segment (start 154.737 94.676) (end 154.888 94.676) (width 0.2) (layer "B.Cu") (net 2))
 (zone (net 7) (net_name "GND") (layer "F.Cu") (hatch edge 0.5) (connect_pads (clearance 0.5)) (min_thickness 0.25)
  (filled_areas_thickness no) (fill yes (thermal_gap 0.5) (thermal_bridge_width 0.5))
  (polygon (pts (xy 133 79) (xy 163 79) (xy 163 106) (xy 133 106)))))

